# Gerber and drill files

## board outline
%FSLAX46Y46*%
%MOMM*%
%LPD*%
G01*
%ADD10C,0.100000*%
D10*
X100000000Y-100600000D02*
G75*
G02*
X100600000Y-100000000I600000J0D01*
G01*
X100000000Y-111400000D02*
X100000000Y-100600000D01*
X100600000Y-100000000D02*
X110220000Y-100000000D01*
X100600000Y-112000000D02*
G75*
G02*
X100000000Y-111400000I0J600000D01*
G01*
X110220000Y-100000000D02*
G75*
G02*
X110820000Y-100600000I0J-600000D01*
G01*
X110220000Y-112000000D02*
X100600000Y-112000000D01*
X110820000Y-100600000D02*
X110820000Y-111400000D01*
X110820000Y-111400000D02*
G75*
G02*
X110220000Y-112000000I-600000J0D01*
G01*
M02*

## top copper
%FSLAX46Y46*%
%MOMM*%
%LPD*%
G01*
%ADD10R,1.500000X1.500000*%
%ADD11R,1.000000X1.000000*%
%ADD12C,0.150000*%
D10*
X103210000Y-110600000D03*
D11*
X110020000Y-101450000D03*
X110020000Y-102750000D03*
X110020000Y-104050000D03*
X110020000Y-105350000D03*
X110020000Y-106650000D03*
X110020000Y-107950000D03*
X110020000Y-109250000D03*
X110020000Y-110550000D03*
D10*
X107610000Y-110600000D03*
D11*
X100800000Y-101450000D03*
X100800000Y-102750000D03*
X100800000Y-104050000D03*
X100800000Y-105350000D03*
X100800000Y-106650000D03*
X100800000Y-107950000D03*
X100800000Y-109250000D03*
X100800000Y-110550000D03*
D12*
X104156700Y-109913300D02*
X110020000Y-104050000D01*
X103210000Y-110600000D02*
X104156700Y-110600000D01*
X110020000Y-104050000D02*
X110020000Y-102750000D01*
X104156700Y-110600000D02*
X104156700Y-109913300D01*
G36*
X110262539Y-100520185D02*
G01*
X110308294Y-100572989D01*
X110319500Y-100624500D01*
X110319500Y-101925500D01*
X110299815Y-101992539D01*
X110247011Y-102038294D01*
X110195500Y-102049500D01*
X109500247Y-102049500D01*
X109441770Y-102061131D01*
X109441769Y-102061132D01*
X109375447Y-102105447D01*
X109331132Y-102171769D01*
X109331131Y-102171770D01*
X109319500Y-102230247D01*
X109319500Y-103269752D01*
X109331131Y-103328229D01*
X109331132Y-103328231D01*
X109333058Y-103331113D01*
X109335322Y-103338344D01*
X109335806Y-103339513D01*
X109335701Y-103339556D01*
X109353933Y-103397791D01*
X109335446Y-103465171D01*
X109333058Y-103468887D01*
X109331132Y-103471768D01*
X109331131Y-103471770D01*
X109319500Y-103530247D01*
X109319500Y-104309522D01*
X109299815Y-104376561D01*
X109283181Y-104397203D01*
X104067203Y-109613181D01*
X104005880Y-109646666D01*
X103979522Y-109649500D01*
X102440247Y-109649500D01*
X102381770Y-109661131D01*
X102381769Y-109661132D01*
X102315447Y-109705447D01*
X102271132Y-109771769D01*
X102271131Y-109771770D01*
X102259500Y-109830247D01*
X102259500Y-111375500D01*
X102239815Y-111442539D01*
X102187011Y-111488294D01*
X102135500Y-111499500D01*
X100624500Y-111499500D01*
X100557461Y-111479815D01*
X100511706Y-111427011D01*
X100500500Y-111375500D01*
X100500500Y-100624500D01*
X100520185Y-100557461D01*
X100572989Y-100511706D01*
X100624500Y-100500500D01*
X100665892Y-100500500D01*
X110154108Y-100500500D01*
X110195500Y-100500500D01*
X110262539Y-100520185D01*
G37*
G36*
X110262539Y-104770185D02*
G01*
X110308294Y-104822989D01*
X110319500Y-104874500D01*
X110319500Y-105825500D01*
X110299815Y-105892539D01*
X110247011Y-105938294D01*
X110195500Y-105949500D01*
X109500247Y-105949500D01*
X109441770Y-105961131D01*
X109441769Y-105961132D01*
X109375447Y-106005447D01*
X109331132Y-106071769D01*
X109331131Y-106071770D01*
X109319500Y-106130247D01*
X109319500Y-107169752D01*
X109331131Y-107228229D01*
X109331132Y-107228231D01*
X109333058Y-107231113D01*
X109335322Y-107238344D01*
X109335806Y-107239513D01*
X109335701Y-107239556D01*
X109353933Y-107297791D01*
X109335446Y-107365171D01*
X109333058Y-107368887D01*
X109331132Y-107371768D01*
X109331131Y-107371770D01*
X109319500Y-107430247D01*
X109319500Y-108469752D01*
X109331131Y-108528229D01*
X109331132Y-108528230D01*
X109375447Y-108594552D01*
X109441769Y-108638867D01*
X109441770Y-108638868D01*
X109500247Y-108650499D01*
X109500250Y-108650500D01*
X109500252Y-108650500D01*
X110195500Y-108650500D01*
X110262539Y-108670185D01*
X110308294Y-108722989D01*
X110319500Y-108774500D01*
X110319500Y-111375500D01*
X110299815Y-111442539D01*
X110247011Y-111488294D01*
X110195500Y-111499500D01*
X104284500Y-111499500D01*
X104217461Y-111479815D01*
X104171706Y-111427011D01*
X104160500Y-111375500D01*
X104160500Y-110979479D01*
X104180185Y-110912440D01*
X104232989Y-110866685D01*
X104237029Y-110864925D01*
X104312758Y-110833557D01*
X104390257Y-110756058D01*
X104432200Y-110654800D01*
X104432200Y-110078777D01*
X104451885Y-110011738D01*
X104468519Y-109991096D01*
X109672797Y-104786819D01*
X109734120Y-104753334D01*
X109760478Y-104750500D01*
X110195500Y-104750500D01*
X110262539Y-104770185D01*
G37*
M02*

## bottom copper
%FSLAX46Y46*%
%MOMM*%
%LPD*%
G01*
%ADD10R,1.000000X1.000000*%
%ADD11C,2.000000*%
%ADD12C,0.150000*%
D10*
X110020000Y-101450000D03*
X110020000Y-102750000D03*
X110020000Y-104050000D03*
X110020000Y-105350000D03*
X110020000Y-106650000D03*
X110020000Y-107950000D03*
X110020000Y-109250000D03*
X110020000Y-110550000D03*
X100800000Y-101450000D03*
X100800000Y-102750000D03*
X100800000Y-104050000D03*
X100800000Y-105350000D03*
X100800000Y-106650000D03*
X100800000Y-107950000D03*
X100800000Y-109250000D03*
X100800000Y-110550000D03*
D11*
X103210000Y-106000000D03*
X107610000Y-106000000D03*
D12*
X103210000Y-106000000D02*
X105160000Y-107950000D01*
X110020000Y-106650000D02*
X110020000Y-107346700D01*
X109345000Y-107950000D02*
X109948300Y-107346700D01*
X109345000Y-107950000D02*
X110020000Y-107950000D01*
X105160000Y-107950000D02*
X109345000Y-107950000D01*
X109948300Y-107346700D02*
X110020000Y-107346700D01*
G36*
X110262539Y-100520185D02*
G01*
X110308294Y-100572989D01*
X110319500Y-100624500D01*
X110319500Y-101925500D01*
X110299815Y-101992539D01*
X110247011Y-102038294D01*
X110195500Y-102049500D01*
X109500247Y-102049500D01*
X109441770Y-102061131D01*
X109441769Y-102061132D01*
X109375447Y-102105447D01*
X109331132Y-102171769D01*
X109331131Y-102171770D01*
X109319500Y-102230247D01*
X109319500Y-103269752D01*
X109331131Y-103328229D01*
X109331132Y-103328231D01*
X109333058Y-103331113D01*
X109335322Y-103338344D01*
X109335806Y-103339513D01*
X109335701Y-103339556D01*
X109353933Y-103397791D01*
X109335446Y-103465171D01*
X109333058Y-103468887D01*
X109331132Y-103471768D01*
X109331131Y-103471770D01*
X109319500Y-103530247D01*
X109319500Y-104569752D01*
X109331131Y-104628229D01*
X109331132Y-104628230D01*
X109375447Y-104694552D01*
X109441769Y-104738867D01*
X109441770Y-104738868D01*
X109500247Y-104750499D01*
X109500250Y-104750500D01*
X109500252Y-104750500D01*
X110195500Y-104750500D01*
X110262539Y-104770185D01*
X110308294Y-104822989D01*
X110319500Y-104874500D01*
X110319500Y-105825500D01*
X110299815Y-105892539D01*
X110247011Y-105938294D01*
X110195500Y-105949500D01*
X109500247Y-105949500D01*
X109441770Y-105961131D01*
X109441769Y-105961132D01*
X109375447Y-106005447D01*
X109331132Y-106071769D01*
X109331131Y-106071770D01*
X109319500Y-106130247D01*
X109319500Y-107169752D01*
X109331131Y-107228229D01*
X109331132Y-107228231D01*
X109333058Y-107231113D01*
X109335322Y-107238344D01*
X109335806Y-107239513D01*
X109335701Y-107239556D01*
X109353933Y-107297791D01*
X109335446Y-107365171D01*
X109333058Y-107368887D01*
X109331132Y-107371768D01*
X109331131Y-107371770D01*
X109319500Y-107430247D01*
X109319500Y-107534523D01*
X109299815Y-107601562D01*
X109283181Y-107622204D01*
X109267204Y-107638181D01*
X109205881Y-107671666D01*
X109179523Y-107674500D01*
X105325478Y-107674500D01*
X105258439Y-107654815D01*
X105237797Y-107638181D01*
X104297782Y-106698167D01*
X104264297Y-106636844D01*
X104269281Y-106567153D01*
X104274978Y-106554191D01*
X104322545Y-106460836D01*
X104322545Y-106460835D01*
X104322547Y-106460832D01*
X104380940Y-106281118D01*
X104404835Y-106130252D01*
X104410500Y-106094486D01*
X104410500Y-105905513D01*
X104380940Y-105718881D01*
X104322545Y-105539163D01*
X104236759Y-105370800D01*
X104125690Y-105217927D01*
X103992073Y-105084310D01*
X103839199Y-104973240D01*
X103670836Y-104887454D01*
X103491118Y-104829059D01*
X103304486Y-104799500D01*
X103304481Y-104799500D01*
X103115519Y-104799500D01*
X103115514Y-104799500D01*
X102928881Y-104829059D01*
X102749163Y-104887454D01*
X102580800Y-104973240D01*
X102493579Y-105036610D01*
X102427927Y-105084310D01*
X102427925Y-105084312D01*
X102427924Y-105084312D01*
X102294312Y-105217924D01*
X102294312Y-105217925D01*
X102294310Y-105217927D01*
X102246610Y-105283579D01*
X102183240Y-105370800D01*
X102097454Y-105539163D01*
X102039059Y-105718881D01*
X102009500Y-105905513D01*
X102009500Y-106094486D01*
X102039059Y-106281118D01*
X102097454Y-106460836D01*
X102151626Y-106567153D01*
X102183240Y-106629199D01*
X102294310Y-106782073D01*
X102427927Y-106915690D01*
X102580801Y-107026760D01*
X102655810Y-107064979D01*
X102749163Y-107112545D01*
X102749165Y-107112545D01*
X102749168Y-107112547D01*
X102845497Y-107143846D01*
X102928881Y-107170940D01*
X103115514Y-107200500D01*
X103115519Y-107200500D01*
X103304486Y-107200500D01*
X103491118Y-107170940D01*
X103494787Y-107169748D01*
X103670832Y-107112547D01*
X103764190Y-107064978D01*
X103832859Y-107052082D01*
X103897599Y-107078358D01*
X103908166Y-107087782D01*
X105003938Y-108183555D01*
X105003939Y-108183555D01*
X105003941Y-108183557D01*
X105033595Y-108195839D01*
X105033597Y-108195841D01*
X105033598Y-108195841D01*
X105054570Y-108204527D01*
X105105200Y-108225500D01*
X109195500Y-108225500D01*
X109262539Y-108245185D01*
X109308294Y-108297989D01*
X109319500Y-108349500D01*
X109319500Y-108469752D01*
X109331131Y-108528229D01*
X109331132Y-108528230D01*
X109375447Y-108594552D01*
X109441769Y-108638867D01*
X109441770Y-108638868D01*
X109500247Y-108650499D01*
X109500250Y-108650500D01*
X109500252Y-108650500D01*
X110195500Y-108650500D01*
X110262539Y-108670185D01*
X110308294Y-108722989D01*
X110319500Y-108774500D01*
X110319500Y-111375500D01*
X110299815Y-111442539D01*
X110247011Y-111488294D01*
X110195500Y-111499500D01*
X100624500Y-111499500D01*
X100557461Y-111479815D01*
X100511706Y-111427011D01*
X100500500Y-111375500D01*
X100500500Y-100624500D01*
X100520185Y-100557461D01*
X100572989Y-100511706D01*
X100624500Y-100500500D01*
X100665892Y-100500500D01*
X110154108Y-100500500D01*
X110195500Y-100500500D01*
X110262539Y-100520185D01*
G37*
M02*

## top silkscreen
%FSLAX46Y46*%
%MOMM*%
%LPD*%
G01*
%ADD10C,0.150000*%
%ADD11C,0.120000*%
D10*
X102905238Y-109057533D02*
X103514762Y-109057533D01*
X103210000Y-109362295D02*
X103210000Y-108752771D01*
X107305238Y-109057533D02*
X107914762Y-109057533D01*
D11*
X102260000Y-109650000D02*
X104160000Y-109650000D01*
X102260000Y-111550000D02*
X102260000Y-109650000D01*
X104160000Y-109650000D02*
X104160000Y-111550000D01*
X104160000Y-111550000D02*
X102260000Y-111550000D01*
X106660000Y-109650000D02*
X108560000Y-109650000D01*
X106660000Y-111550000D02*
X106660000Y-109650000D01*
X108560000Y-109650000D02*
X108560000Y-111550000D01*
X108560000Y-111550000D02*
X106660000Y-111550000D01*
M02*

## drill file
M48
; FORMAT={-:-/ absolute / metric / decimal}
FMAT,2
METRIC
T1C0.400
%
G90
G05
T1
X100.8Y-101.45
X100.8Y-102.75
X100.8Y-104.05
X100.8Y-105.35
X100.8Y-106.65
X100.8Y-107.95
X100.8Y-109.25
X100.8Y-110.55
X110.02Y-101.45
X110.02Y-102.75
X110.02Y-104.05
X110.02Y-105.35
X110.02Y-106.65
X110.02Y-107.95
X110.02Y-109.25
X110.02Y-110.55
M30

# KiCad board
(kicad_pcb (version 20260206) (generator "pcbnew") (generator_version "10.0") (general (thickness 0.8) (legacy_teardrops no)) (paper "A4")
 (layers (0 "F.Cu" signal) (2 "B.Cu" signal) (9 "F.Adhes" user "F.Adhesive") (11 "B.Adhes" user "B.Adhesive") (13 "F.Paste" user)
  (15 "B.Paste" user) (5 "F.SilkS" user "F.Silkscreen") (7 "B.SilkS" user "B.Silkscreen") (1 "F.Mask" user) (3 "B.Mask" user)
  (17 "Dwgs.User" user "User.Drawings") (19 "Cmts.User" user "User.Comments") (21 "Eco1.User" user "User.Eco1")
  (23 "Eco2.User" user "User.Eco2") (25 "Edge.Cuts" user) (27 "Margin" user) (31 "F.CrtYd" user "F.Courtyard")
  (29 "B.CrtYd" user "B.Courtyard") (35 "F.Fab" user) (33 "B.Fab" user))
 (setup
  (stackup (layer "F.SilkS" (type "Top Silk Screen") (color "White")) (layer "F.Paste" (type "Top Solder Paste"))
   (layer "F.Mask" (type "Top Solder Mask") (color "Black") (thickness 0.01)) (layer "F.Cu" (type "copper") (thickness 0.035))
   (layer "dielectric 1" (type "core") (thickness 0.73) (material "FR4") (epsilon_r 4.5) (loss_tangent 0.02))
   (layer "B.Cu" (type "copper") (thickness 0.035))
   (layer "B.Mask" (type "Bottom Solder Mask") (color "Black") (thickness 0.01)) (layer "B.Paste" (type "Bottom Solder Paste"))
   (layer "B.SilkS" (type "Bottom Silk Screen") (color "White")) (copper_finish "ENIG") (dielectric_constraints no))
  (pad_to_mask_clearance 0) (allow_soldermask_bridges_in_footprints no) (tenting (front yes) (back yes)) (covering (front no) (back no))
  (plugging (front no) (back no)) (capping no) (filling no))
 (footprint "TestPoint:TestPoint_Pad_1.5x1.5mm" (layer "F.Cu") (at 103.21 110.6)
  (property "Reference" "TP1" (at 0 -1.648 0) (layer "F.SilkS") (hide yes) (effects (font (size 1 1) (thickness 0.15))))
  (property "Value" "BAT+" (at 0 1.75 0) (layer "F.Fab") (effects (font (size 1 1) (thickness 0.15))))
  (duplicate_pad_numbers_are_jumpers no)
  (fp_line (start -0.95 -0.95) (end 0.95 -0.95) (stroke (width 0.12) (type solid)) (layer "F.SilkS"))
  (fp_line (start -0.95 0.95) (end -0.95 -0.95) (stroke (width 0.12) (type solid)) (layer "F.SilkS"))
  (fp_line (start 0.95 -0.95) (end 0.95 0.95) (stroke (width 0.12) (type solid)) (layer "F.SilkS"))
  (fp_line (start 0.95 0.95) (end -0.95 0.95) (stroke (width 0.12) (type solid)) (layer "F.SilkS"))
  (pad "1" smd rect (at 0 0) (size 1.5 1.5) (layers "F.Cu" "F.Mask") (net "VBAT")))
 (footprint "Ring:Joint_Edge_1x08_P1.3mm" (layer "F.Cu") (at 110.02 106)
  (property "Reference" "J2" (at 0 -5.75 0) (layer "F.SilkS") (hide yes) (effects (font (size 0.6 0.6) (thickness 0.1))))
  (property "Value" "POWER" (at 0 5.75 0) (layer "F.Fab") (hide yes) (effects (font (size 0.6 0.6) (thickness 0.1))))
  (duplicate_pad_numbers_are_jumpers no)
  (pad "1" thru_hole rect (at 0 -4.55) (size 1 1) (drill 0.4) (layers "*.Cu" "*.Mask") (remove_unused_layers no) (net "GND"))
  (pad "2" thru_hole rect (at 0 -3.25) (size 1 1) (drill 0.4) (layers "*.Cu" "*.Mask") (remove_unused_layers no) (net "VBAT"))
  (pad "3" thru_hole rect (at 0 -1.95) (size 1 1) (drill 0.4) (layers "*.Cu" "*.Mask") (remove_unused_layers no) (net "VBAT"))
  (pad "4" thru_hole rect (at 0 -0.65) (size 1 1) (drill 0.4) (layers "*.Cu" "*.Mask") (remove_unused_layers no) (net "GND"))
  (pad "5" thru_hole rect (at 0 0.65) (size 1 1) (drill 0.4) (layers "*.Cu" "*.Mask") (remove_unused_layers no) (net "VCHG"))
  (pad "6" thru_hole rect (at 0 1.95) (size 1 1) (drill 0.4) (layers "*.Cu" "*.Mask") (remove_unused_layers no) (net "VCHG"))
  (pad "7" thru_hole rect (at 0 3.25) (size 1 1) (drill 0.4) (layers "*.Cu" "*.Mask") (remove_unused_layers no) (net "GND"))
  (pad "8" thru_hole rect (at 0 4.55) (size 1 1) (drill 0.4) (layers "*.Cu" "*.Mask") (remove_unused_layers no) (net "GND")))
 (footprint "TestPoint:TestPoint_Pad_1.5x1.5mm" (layer "F.Cu") (at 107.61 110.6)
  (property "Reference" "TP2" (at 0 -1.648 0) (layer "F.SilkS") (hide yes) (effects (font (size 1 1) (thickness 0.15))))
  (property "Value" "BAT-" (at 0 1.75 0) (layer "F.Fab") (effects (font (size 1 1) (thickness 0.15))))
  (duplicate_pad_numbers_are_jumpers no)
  (fp_line (start -0.95 -0.95) (end 0.95 -0.95) (stroke (width 0.12) (type solid)) (layer "F.SilkS"))
  (fp_line (start -0.95 0.95) (end -0.95 -0.95) (stroke (width 0.12) (type solid)) (layer "F.SilkS"))
  (fp_line (start 0.95 -0.95) (end 0.95 0.95) (stroke (width 0.12) (type solid)) (layer "F.SilkS"))
  (fp_line (start 0.95 0.95) (end -0.95 0.95) (stroke (width 0.12) (type solid)) (layer "F.SilkS"))
  (pad "1" smd rect (at 0 0) (size 1.5 1.5) (layers "F.Cu" "F.Mask") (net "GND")))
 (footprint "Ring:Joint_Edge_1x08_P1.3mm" (layer "F.Cu") (at 100.8 106)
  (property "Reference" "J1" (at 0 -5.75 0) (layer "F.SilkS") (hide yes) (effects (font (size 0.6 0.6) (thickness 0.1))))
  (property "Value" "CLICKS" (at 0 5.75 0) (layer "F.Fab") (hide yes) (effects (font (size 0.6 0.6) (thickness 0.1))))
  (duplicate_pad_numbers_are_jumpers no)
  (pad "1" thru_hole rect (at 0 -4.55) (size 1 1) (drill 0.4) (layers "*.Cu" "*.Mask") (remove_unused_layers no) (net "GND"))
  (pad "2" thru_hole rect (at 0 -3.25) (size 1 1) (drill 0.4) (layers "*.Cu" "*.Mask") (remove_unused_layers no) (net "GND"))
  (pad "3" thru_hole rect (at 0 -1.95) (size 1 1) (drill 0.4) (layers "*.Cu" "*.Mask") (remove_unused_layers no) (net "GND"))
  (pad "4" thru_hole rect (at 0 -0.65) (size 1 1) (drill 0.4) (layers "*.Cu" "*.Mask") (remove_unused_layers no) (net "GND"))
  (pad "5" thru_hole rect (at 0 0.65) (size 1 1) (drill 0.4) (layers "*.Cu" "*.Mask") (remove_unused_layers no) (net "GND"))
  (pad "6" thru_hole rect (at 0 1.95) (size 1 1) (drill 0.4) (layers "*.Cu" "*.Mask") (remove_unused_layers no) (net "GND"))
  (pad "7" thru_hole rect (at 0 3.25) (size 1 1) (drill 0.4) (layers "*.Cu" "*.Mask") (remove_unused_layers no) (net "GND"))
  (pad "8" thru_hole rect (at 0 4.55) (size 1 1) (drill 0.4) (layers "*.Cu" "*.Mask") (remove_unused_layers no) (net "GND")))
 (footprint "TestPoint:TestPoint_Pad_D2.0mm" (layer "B.Cu") (at 103.21 106)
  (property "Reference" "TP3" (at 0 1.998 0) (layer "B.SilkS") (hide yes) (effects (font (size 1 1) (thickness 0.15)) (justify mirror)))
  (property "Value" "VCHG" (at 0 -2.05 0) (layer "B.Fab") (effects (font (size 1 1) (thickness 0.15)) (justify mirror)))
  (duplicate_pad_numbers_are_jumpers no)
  (pad "1" smd circle (at 0 0) (size 2 2) (layers "B.Cu" "B.Mask") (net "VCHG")))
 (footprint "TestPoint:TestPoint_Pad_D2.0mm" (layer "B.Cu") (at 107.61 106)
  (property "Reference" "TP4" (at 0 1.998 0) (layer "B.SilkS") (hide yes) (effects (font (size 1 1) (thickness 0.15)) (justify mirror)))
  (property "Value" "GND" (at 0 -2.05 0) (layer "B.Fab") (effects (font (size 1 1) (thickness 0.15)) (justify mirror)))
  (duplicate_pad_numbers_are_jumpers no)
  (pad "1" smd circle (at 0 0) (size 2 2) (layers "B.Cu" "B.Mask") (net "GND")))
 (gr_arc (start 100 100.6) (mid 100.175736 100.175736) (end 100.6 100) (stroke (width 0.1) (type default)) (layer "Edge.Cuts"))
 (gr_line (start 100 111.4) (end 100 100.6) (stroke (width 0.1) (type default)) (layer "Edge.Cuts"))
 (gr_line (start 100.6 100) (end 110.22 100) (stroke (width 0.1) (type default)) (layer "Edge.Cuts"))
 (gr_arc (start 100.6 112) (mid 100.175736 111.824264) (end 100 111.4) (stroke (width 0.1) (type default)) (layer "Edge.Cuts"))
 (gr_arc (start 110.22 100) (mid 110.644264 100.175736) (end 110.82 100.6) (stroke (width 0.1) (type default)) (layer "Edge.Cuts"))
 (gr_line (start 110.22 112) (end 100.6 112) (stroke (width 0.1) (type default)) (layer "Edge.Cuts"))
 (gr_line (start 110.82 100.6) (end 110.82 111.4) (stroke (width 0.1) (type default)) (layer "Edge.Cuts"))
 (gr_arc (start 110.82 111.4) (mid 110.644264 111.824264) (end 110.22 112) (stroke (width 0.1) (type default)) (layer "Edge.Cuts"))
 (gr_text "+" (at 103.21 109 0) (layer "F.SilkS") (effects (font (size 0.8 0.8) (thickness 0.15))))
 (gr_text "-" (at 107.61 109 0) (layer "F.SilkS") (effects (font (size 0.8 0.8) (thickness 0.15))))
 (segment (start 104.1567 109.9133) (end 110.02 104.05) (width 0.15) (layer "F.Cu") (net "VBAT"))
 (segment (start 103.21 110.6) (end 104.1567 110.6) (width 0.15) (layer "F.Cu") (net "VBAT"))
 (segment (start 110.02 104.05) (end 110.02 102.75) (width 0.15) (layer "F.Cu") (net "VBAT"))
 (segment (start 104.1567 110.6) (end 104.1567 109.9133) (width 0.15) (layer "F.Cu") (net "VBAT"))
 (segment (start 103.21 106) (end 105.16 107.95) (width 0.15) (layer "B.Cu") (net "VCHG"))
 (segment (start 110.02 106.65) (end 110.02 107.3467) (width 0.15) (layer "B.Cu") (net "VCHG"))
 (segment (start 109.345 107.95) (end 109.9483 107.3467) (width 0.15) (layer "B.Cu") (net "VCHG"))
 (segment (start 109.345 107.95) (end 110.02 107.95) (width 0.15) (layer "B.Cu") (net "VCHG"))
 (segment (start 105.16 107.95) (end 109.345 107.95) (width 0.15) (layer "B.Cu") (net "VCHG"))
 (segment (start 109.9483 107.3467) (end 110.02 107.3467) (width 0.15) (layer "B.Cu") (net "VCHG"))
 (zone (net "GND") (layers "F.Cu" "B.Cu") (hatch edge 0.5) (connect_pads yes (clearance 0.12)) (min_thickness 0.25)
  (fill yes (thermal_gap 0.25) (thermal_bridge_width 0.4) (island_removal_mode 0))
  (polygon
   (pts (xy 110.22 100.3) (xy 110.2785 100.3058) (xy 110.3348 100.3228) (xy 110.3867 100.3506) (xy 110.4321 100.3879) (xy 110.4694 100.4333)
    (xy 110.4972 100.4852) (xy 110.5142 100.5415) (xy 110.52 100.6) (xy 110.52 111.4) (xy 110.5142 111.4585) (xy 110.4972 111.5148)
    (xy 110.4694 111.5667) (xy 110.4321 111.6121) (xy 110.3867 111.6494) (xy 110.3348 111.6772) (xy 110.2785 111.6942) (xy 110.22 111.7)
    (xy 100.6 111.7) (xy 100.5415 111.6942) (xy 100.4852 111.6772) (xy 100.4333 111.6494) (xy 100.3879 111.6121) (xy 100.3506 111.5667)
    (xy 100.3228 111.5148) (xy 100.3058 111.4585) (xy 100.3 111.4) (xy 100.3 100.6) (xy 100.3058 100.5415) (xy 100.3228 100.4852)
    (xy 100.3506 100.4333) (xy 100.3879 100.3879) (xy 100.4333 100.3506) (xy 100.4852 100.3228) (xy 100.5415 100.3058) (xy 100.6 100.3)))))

